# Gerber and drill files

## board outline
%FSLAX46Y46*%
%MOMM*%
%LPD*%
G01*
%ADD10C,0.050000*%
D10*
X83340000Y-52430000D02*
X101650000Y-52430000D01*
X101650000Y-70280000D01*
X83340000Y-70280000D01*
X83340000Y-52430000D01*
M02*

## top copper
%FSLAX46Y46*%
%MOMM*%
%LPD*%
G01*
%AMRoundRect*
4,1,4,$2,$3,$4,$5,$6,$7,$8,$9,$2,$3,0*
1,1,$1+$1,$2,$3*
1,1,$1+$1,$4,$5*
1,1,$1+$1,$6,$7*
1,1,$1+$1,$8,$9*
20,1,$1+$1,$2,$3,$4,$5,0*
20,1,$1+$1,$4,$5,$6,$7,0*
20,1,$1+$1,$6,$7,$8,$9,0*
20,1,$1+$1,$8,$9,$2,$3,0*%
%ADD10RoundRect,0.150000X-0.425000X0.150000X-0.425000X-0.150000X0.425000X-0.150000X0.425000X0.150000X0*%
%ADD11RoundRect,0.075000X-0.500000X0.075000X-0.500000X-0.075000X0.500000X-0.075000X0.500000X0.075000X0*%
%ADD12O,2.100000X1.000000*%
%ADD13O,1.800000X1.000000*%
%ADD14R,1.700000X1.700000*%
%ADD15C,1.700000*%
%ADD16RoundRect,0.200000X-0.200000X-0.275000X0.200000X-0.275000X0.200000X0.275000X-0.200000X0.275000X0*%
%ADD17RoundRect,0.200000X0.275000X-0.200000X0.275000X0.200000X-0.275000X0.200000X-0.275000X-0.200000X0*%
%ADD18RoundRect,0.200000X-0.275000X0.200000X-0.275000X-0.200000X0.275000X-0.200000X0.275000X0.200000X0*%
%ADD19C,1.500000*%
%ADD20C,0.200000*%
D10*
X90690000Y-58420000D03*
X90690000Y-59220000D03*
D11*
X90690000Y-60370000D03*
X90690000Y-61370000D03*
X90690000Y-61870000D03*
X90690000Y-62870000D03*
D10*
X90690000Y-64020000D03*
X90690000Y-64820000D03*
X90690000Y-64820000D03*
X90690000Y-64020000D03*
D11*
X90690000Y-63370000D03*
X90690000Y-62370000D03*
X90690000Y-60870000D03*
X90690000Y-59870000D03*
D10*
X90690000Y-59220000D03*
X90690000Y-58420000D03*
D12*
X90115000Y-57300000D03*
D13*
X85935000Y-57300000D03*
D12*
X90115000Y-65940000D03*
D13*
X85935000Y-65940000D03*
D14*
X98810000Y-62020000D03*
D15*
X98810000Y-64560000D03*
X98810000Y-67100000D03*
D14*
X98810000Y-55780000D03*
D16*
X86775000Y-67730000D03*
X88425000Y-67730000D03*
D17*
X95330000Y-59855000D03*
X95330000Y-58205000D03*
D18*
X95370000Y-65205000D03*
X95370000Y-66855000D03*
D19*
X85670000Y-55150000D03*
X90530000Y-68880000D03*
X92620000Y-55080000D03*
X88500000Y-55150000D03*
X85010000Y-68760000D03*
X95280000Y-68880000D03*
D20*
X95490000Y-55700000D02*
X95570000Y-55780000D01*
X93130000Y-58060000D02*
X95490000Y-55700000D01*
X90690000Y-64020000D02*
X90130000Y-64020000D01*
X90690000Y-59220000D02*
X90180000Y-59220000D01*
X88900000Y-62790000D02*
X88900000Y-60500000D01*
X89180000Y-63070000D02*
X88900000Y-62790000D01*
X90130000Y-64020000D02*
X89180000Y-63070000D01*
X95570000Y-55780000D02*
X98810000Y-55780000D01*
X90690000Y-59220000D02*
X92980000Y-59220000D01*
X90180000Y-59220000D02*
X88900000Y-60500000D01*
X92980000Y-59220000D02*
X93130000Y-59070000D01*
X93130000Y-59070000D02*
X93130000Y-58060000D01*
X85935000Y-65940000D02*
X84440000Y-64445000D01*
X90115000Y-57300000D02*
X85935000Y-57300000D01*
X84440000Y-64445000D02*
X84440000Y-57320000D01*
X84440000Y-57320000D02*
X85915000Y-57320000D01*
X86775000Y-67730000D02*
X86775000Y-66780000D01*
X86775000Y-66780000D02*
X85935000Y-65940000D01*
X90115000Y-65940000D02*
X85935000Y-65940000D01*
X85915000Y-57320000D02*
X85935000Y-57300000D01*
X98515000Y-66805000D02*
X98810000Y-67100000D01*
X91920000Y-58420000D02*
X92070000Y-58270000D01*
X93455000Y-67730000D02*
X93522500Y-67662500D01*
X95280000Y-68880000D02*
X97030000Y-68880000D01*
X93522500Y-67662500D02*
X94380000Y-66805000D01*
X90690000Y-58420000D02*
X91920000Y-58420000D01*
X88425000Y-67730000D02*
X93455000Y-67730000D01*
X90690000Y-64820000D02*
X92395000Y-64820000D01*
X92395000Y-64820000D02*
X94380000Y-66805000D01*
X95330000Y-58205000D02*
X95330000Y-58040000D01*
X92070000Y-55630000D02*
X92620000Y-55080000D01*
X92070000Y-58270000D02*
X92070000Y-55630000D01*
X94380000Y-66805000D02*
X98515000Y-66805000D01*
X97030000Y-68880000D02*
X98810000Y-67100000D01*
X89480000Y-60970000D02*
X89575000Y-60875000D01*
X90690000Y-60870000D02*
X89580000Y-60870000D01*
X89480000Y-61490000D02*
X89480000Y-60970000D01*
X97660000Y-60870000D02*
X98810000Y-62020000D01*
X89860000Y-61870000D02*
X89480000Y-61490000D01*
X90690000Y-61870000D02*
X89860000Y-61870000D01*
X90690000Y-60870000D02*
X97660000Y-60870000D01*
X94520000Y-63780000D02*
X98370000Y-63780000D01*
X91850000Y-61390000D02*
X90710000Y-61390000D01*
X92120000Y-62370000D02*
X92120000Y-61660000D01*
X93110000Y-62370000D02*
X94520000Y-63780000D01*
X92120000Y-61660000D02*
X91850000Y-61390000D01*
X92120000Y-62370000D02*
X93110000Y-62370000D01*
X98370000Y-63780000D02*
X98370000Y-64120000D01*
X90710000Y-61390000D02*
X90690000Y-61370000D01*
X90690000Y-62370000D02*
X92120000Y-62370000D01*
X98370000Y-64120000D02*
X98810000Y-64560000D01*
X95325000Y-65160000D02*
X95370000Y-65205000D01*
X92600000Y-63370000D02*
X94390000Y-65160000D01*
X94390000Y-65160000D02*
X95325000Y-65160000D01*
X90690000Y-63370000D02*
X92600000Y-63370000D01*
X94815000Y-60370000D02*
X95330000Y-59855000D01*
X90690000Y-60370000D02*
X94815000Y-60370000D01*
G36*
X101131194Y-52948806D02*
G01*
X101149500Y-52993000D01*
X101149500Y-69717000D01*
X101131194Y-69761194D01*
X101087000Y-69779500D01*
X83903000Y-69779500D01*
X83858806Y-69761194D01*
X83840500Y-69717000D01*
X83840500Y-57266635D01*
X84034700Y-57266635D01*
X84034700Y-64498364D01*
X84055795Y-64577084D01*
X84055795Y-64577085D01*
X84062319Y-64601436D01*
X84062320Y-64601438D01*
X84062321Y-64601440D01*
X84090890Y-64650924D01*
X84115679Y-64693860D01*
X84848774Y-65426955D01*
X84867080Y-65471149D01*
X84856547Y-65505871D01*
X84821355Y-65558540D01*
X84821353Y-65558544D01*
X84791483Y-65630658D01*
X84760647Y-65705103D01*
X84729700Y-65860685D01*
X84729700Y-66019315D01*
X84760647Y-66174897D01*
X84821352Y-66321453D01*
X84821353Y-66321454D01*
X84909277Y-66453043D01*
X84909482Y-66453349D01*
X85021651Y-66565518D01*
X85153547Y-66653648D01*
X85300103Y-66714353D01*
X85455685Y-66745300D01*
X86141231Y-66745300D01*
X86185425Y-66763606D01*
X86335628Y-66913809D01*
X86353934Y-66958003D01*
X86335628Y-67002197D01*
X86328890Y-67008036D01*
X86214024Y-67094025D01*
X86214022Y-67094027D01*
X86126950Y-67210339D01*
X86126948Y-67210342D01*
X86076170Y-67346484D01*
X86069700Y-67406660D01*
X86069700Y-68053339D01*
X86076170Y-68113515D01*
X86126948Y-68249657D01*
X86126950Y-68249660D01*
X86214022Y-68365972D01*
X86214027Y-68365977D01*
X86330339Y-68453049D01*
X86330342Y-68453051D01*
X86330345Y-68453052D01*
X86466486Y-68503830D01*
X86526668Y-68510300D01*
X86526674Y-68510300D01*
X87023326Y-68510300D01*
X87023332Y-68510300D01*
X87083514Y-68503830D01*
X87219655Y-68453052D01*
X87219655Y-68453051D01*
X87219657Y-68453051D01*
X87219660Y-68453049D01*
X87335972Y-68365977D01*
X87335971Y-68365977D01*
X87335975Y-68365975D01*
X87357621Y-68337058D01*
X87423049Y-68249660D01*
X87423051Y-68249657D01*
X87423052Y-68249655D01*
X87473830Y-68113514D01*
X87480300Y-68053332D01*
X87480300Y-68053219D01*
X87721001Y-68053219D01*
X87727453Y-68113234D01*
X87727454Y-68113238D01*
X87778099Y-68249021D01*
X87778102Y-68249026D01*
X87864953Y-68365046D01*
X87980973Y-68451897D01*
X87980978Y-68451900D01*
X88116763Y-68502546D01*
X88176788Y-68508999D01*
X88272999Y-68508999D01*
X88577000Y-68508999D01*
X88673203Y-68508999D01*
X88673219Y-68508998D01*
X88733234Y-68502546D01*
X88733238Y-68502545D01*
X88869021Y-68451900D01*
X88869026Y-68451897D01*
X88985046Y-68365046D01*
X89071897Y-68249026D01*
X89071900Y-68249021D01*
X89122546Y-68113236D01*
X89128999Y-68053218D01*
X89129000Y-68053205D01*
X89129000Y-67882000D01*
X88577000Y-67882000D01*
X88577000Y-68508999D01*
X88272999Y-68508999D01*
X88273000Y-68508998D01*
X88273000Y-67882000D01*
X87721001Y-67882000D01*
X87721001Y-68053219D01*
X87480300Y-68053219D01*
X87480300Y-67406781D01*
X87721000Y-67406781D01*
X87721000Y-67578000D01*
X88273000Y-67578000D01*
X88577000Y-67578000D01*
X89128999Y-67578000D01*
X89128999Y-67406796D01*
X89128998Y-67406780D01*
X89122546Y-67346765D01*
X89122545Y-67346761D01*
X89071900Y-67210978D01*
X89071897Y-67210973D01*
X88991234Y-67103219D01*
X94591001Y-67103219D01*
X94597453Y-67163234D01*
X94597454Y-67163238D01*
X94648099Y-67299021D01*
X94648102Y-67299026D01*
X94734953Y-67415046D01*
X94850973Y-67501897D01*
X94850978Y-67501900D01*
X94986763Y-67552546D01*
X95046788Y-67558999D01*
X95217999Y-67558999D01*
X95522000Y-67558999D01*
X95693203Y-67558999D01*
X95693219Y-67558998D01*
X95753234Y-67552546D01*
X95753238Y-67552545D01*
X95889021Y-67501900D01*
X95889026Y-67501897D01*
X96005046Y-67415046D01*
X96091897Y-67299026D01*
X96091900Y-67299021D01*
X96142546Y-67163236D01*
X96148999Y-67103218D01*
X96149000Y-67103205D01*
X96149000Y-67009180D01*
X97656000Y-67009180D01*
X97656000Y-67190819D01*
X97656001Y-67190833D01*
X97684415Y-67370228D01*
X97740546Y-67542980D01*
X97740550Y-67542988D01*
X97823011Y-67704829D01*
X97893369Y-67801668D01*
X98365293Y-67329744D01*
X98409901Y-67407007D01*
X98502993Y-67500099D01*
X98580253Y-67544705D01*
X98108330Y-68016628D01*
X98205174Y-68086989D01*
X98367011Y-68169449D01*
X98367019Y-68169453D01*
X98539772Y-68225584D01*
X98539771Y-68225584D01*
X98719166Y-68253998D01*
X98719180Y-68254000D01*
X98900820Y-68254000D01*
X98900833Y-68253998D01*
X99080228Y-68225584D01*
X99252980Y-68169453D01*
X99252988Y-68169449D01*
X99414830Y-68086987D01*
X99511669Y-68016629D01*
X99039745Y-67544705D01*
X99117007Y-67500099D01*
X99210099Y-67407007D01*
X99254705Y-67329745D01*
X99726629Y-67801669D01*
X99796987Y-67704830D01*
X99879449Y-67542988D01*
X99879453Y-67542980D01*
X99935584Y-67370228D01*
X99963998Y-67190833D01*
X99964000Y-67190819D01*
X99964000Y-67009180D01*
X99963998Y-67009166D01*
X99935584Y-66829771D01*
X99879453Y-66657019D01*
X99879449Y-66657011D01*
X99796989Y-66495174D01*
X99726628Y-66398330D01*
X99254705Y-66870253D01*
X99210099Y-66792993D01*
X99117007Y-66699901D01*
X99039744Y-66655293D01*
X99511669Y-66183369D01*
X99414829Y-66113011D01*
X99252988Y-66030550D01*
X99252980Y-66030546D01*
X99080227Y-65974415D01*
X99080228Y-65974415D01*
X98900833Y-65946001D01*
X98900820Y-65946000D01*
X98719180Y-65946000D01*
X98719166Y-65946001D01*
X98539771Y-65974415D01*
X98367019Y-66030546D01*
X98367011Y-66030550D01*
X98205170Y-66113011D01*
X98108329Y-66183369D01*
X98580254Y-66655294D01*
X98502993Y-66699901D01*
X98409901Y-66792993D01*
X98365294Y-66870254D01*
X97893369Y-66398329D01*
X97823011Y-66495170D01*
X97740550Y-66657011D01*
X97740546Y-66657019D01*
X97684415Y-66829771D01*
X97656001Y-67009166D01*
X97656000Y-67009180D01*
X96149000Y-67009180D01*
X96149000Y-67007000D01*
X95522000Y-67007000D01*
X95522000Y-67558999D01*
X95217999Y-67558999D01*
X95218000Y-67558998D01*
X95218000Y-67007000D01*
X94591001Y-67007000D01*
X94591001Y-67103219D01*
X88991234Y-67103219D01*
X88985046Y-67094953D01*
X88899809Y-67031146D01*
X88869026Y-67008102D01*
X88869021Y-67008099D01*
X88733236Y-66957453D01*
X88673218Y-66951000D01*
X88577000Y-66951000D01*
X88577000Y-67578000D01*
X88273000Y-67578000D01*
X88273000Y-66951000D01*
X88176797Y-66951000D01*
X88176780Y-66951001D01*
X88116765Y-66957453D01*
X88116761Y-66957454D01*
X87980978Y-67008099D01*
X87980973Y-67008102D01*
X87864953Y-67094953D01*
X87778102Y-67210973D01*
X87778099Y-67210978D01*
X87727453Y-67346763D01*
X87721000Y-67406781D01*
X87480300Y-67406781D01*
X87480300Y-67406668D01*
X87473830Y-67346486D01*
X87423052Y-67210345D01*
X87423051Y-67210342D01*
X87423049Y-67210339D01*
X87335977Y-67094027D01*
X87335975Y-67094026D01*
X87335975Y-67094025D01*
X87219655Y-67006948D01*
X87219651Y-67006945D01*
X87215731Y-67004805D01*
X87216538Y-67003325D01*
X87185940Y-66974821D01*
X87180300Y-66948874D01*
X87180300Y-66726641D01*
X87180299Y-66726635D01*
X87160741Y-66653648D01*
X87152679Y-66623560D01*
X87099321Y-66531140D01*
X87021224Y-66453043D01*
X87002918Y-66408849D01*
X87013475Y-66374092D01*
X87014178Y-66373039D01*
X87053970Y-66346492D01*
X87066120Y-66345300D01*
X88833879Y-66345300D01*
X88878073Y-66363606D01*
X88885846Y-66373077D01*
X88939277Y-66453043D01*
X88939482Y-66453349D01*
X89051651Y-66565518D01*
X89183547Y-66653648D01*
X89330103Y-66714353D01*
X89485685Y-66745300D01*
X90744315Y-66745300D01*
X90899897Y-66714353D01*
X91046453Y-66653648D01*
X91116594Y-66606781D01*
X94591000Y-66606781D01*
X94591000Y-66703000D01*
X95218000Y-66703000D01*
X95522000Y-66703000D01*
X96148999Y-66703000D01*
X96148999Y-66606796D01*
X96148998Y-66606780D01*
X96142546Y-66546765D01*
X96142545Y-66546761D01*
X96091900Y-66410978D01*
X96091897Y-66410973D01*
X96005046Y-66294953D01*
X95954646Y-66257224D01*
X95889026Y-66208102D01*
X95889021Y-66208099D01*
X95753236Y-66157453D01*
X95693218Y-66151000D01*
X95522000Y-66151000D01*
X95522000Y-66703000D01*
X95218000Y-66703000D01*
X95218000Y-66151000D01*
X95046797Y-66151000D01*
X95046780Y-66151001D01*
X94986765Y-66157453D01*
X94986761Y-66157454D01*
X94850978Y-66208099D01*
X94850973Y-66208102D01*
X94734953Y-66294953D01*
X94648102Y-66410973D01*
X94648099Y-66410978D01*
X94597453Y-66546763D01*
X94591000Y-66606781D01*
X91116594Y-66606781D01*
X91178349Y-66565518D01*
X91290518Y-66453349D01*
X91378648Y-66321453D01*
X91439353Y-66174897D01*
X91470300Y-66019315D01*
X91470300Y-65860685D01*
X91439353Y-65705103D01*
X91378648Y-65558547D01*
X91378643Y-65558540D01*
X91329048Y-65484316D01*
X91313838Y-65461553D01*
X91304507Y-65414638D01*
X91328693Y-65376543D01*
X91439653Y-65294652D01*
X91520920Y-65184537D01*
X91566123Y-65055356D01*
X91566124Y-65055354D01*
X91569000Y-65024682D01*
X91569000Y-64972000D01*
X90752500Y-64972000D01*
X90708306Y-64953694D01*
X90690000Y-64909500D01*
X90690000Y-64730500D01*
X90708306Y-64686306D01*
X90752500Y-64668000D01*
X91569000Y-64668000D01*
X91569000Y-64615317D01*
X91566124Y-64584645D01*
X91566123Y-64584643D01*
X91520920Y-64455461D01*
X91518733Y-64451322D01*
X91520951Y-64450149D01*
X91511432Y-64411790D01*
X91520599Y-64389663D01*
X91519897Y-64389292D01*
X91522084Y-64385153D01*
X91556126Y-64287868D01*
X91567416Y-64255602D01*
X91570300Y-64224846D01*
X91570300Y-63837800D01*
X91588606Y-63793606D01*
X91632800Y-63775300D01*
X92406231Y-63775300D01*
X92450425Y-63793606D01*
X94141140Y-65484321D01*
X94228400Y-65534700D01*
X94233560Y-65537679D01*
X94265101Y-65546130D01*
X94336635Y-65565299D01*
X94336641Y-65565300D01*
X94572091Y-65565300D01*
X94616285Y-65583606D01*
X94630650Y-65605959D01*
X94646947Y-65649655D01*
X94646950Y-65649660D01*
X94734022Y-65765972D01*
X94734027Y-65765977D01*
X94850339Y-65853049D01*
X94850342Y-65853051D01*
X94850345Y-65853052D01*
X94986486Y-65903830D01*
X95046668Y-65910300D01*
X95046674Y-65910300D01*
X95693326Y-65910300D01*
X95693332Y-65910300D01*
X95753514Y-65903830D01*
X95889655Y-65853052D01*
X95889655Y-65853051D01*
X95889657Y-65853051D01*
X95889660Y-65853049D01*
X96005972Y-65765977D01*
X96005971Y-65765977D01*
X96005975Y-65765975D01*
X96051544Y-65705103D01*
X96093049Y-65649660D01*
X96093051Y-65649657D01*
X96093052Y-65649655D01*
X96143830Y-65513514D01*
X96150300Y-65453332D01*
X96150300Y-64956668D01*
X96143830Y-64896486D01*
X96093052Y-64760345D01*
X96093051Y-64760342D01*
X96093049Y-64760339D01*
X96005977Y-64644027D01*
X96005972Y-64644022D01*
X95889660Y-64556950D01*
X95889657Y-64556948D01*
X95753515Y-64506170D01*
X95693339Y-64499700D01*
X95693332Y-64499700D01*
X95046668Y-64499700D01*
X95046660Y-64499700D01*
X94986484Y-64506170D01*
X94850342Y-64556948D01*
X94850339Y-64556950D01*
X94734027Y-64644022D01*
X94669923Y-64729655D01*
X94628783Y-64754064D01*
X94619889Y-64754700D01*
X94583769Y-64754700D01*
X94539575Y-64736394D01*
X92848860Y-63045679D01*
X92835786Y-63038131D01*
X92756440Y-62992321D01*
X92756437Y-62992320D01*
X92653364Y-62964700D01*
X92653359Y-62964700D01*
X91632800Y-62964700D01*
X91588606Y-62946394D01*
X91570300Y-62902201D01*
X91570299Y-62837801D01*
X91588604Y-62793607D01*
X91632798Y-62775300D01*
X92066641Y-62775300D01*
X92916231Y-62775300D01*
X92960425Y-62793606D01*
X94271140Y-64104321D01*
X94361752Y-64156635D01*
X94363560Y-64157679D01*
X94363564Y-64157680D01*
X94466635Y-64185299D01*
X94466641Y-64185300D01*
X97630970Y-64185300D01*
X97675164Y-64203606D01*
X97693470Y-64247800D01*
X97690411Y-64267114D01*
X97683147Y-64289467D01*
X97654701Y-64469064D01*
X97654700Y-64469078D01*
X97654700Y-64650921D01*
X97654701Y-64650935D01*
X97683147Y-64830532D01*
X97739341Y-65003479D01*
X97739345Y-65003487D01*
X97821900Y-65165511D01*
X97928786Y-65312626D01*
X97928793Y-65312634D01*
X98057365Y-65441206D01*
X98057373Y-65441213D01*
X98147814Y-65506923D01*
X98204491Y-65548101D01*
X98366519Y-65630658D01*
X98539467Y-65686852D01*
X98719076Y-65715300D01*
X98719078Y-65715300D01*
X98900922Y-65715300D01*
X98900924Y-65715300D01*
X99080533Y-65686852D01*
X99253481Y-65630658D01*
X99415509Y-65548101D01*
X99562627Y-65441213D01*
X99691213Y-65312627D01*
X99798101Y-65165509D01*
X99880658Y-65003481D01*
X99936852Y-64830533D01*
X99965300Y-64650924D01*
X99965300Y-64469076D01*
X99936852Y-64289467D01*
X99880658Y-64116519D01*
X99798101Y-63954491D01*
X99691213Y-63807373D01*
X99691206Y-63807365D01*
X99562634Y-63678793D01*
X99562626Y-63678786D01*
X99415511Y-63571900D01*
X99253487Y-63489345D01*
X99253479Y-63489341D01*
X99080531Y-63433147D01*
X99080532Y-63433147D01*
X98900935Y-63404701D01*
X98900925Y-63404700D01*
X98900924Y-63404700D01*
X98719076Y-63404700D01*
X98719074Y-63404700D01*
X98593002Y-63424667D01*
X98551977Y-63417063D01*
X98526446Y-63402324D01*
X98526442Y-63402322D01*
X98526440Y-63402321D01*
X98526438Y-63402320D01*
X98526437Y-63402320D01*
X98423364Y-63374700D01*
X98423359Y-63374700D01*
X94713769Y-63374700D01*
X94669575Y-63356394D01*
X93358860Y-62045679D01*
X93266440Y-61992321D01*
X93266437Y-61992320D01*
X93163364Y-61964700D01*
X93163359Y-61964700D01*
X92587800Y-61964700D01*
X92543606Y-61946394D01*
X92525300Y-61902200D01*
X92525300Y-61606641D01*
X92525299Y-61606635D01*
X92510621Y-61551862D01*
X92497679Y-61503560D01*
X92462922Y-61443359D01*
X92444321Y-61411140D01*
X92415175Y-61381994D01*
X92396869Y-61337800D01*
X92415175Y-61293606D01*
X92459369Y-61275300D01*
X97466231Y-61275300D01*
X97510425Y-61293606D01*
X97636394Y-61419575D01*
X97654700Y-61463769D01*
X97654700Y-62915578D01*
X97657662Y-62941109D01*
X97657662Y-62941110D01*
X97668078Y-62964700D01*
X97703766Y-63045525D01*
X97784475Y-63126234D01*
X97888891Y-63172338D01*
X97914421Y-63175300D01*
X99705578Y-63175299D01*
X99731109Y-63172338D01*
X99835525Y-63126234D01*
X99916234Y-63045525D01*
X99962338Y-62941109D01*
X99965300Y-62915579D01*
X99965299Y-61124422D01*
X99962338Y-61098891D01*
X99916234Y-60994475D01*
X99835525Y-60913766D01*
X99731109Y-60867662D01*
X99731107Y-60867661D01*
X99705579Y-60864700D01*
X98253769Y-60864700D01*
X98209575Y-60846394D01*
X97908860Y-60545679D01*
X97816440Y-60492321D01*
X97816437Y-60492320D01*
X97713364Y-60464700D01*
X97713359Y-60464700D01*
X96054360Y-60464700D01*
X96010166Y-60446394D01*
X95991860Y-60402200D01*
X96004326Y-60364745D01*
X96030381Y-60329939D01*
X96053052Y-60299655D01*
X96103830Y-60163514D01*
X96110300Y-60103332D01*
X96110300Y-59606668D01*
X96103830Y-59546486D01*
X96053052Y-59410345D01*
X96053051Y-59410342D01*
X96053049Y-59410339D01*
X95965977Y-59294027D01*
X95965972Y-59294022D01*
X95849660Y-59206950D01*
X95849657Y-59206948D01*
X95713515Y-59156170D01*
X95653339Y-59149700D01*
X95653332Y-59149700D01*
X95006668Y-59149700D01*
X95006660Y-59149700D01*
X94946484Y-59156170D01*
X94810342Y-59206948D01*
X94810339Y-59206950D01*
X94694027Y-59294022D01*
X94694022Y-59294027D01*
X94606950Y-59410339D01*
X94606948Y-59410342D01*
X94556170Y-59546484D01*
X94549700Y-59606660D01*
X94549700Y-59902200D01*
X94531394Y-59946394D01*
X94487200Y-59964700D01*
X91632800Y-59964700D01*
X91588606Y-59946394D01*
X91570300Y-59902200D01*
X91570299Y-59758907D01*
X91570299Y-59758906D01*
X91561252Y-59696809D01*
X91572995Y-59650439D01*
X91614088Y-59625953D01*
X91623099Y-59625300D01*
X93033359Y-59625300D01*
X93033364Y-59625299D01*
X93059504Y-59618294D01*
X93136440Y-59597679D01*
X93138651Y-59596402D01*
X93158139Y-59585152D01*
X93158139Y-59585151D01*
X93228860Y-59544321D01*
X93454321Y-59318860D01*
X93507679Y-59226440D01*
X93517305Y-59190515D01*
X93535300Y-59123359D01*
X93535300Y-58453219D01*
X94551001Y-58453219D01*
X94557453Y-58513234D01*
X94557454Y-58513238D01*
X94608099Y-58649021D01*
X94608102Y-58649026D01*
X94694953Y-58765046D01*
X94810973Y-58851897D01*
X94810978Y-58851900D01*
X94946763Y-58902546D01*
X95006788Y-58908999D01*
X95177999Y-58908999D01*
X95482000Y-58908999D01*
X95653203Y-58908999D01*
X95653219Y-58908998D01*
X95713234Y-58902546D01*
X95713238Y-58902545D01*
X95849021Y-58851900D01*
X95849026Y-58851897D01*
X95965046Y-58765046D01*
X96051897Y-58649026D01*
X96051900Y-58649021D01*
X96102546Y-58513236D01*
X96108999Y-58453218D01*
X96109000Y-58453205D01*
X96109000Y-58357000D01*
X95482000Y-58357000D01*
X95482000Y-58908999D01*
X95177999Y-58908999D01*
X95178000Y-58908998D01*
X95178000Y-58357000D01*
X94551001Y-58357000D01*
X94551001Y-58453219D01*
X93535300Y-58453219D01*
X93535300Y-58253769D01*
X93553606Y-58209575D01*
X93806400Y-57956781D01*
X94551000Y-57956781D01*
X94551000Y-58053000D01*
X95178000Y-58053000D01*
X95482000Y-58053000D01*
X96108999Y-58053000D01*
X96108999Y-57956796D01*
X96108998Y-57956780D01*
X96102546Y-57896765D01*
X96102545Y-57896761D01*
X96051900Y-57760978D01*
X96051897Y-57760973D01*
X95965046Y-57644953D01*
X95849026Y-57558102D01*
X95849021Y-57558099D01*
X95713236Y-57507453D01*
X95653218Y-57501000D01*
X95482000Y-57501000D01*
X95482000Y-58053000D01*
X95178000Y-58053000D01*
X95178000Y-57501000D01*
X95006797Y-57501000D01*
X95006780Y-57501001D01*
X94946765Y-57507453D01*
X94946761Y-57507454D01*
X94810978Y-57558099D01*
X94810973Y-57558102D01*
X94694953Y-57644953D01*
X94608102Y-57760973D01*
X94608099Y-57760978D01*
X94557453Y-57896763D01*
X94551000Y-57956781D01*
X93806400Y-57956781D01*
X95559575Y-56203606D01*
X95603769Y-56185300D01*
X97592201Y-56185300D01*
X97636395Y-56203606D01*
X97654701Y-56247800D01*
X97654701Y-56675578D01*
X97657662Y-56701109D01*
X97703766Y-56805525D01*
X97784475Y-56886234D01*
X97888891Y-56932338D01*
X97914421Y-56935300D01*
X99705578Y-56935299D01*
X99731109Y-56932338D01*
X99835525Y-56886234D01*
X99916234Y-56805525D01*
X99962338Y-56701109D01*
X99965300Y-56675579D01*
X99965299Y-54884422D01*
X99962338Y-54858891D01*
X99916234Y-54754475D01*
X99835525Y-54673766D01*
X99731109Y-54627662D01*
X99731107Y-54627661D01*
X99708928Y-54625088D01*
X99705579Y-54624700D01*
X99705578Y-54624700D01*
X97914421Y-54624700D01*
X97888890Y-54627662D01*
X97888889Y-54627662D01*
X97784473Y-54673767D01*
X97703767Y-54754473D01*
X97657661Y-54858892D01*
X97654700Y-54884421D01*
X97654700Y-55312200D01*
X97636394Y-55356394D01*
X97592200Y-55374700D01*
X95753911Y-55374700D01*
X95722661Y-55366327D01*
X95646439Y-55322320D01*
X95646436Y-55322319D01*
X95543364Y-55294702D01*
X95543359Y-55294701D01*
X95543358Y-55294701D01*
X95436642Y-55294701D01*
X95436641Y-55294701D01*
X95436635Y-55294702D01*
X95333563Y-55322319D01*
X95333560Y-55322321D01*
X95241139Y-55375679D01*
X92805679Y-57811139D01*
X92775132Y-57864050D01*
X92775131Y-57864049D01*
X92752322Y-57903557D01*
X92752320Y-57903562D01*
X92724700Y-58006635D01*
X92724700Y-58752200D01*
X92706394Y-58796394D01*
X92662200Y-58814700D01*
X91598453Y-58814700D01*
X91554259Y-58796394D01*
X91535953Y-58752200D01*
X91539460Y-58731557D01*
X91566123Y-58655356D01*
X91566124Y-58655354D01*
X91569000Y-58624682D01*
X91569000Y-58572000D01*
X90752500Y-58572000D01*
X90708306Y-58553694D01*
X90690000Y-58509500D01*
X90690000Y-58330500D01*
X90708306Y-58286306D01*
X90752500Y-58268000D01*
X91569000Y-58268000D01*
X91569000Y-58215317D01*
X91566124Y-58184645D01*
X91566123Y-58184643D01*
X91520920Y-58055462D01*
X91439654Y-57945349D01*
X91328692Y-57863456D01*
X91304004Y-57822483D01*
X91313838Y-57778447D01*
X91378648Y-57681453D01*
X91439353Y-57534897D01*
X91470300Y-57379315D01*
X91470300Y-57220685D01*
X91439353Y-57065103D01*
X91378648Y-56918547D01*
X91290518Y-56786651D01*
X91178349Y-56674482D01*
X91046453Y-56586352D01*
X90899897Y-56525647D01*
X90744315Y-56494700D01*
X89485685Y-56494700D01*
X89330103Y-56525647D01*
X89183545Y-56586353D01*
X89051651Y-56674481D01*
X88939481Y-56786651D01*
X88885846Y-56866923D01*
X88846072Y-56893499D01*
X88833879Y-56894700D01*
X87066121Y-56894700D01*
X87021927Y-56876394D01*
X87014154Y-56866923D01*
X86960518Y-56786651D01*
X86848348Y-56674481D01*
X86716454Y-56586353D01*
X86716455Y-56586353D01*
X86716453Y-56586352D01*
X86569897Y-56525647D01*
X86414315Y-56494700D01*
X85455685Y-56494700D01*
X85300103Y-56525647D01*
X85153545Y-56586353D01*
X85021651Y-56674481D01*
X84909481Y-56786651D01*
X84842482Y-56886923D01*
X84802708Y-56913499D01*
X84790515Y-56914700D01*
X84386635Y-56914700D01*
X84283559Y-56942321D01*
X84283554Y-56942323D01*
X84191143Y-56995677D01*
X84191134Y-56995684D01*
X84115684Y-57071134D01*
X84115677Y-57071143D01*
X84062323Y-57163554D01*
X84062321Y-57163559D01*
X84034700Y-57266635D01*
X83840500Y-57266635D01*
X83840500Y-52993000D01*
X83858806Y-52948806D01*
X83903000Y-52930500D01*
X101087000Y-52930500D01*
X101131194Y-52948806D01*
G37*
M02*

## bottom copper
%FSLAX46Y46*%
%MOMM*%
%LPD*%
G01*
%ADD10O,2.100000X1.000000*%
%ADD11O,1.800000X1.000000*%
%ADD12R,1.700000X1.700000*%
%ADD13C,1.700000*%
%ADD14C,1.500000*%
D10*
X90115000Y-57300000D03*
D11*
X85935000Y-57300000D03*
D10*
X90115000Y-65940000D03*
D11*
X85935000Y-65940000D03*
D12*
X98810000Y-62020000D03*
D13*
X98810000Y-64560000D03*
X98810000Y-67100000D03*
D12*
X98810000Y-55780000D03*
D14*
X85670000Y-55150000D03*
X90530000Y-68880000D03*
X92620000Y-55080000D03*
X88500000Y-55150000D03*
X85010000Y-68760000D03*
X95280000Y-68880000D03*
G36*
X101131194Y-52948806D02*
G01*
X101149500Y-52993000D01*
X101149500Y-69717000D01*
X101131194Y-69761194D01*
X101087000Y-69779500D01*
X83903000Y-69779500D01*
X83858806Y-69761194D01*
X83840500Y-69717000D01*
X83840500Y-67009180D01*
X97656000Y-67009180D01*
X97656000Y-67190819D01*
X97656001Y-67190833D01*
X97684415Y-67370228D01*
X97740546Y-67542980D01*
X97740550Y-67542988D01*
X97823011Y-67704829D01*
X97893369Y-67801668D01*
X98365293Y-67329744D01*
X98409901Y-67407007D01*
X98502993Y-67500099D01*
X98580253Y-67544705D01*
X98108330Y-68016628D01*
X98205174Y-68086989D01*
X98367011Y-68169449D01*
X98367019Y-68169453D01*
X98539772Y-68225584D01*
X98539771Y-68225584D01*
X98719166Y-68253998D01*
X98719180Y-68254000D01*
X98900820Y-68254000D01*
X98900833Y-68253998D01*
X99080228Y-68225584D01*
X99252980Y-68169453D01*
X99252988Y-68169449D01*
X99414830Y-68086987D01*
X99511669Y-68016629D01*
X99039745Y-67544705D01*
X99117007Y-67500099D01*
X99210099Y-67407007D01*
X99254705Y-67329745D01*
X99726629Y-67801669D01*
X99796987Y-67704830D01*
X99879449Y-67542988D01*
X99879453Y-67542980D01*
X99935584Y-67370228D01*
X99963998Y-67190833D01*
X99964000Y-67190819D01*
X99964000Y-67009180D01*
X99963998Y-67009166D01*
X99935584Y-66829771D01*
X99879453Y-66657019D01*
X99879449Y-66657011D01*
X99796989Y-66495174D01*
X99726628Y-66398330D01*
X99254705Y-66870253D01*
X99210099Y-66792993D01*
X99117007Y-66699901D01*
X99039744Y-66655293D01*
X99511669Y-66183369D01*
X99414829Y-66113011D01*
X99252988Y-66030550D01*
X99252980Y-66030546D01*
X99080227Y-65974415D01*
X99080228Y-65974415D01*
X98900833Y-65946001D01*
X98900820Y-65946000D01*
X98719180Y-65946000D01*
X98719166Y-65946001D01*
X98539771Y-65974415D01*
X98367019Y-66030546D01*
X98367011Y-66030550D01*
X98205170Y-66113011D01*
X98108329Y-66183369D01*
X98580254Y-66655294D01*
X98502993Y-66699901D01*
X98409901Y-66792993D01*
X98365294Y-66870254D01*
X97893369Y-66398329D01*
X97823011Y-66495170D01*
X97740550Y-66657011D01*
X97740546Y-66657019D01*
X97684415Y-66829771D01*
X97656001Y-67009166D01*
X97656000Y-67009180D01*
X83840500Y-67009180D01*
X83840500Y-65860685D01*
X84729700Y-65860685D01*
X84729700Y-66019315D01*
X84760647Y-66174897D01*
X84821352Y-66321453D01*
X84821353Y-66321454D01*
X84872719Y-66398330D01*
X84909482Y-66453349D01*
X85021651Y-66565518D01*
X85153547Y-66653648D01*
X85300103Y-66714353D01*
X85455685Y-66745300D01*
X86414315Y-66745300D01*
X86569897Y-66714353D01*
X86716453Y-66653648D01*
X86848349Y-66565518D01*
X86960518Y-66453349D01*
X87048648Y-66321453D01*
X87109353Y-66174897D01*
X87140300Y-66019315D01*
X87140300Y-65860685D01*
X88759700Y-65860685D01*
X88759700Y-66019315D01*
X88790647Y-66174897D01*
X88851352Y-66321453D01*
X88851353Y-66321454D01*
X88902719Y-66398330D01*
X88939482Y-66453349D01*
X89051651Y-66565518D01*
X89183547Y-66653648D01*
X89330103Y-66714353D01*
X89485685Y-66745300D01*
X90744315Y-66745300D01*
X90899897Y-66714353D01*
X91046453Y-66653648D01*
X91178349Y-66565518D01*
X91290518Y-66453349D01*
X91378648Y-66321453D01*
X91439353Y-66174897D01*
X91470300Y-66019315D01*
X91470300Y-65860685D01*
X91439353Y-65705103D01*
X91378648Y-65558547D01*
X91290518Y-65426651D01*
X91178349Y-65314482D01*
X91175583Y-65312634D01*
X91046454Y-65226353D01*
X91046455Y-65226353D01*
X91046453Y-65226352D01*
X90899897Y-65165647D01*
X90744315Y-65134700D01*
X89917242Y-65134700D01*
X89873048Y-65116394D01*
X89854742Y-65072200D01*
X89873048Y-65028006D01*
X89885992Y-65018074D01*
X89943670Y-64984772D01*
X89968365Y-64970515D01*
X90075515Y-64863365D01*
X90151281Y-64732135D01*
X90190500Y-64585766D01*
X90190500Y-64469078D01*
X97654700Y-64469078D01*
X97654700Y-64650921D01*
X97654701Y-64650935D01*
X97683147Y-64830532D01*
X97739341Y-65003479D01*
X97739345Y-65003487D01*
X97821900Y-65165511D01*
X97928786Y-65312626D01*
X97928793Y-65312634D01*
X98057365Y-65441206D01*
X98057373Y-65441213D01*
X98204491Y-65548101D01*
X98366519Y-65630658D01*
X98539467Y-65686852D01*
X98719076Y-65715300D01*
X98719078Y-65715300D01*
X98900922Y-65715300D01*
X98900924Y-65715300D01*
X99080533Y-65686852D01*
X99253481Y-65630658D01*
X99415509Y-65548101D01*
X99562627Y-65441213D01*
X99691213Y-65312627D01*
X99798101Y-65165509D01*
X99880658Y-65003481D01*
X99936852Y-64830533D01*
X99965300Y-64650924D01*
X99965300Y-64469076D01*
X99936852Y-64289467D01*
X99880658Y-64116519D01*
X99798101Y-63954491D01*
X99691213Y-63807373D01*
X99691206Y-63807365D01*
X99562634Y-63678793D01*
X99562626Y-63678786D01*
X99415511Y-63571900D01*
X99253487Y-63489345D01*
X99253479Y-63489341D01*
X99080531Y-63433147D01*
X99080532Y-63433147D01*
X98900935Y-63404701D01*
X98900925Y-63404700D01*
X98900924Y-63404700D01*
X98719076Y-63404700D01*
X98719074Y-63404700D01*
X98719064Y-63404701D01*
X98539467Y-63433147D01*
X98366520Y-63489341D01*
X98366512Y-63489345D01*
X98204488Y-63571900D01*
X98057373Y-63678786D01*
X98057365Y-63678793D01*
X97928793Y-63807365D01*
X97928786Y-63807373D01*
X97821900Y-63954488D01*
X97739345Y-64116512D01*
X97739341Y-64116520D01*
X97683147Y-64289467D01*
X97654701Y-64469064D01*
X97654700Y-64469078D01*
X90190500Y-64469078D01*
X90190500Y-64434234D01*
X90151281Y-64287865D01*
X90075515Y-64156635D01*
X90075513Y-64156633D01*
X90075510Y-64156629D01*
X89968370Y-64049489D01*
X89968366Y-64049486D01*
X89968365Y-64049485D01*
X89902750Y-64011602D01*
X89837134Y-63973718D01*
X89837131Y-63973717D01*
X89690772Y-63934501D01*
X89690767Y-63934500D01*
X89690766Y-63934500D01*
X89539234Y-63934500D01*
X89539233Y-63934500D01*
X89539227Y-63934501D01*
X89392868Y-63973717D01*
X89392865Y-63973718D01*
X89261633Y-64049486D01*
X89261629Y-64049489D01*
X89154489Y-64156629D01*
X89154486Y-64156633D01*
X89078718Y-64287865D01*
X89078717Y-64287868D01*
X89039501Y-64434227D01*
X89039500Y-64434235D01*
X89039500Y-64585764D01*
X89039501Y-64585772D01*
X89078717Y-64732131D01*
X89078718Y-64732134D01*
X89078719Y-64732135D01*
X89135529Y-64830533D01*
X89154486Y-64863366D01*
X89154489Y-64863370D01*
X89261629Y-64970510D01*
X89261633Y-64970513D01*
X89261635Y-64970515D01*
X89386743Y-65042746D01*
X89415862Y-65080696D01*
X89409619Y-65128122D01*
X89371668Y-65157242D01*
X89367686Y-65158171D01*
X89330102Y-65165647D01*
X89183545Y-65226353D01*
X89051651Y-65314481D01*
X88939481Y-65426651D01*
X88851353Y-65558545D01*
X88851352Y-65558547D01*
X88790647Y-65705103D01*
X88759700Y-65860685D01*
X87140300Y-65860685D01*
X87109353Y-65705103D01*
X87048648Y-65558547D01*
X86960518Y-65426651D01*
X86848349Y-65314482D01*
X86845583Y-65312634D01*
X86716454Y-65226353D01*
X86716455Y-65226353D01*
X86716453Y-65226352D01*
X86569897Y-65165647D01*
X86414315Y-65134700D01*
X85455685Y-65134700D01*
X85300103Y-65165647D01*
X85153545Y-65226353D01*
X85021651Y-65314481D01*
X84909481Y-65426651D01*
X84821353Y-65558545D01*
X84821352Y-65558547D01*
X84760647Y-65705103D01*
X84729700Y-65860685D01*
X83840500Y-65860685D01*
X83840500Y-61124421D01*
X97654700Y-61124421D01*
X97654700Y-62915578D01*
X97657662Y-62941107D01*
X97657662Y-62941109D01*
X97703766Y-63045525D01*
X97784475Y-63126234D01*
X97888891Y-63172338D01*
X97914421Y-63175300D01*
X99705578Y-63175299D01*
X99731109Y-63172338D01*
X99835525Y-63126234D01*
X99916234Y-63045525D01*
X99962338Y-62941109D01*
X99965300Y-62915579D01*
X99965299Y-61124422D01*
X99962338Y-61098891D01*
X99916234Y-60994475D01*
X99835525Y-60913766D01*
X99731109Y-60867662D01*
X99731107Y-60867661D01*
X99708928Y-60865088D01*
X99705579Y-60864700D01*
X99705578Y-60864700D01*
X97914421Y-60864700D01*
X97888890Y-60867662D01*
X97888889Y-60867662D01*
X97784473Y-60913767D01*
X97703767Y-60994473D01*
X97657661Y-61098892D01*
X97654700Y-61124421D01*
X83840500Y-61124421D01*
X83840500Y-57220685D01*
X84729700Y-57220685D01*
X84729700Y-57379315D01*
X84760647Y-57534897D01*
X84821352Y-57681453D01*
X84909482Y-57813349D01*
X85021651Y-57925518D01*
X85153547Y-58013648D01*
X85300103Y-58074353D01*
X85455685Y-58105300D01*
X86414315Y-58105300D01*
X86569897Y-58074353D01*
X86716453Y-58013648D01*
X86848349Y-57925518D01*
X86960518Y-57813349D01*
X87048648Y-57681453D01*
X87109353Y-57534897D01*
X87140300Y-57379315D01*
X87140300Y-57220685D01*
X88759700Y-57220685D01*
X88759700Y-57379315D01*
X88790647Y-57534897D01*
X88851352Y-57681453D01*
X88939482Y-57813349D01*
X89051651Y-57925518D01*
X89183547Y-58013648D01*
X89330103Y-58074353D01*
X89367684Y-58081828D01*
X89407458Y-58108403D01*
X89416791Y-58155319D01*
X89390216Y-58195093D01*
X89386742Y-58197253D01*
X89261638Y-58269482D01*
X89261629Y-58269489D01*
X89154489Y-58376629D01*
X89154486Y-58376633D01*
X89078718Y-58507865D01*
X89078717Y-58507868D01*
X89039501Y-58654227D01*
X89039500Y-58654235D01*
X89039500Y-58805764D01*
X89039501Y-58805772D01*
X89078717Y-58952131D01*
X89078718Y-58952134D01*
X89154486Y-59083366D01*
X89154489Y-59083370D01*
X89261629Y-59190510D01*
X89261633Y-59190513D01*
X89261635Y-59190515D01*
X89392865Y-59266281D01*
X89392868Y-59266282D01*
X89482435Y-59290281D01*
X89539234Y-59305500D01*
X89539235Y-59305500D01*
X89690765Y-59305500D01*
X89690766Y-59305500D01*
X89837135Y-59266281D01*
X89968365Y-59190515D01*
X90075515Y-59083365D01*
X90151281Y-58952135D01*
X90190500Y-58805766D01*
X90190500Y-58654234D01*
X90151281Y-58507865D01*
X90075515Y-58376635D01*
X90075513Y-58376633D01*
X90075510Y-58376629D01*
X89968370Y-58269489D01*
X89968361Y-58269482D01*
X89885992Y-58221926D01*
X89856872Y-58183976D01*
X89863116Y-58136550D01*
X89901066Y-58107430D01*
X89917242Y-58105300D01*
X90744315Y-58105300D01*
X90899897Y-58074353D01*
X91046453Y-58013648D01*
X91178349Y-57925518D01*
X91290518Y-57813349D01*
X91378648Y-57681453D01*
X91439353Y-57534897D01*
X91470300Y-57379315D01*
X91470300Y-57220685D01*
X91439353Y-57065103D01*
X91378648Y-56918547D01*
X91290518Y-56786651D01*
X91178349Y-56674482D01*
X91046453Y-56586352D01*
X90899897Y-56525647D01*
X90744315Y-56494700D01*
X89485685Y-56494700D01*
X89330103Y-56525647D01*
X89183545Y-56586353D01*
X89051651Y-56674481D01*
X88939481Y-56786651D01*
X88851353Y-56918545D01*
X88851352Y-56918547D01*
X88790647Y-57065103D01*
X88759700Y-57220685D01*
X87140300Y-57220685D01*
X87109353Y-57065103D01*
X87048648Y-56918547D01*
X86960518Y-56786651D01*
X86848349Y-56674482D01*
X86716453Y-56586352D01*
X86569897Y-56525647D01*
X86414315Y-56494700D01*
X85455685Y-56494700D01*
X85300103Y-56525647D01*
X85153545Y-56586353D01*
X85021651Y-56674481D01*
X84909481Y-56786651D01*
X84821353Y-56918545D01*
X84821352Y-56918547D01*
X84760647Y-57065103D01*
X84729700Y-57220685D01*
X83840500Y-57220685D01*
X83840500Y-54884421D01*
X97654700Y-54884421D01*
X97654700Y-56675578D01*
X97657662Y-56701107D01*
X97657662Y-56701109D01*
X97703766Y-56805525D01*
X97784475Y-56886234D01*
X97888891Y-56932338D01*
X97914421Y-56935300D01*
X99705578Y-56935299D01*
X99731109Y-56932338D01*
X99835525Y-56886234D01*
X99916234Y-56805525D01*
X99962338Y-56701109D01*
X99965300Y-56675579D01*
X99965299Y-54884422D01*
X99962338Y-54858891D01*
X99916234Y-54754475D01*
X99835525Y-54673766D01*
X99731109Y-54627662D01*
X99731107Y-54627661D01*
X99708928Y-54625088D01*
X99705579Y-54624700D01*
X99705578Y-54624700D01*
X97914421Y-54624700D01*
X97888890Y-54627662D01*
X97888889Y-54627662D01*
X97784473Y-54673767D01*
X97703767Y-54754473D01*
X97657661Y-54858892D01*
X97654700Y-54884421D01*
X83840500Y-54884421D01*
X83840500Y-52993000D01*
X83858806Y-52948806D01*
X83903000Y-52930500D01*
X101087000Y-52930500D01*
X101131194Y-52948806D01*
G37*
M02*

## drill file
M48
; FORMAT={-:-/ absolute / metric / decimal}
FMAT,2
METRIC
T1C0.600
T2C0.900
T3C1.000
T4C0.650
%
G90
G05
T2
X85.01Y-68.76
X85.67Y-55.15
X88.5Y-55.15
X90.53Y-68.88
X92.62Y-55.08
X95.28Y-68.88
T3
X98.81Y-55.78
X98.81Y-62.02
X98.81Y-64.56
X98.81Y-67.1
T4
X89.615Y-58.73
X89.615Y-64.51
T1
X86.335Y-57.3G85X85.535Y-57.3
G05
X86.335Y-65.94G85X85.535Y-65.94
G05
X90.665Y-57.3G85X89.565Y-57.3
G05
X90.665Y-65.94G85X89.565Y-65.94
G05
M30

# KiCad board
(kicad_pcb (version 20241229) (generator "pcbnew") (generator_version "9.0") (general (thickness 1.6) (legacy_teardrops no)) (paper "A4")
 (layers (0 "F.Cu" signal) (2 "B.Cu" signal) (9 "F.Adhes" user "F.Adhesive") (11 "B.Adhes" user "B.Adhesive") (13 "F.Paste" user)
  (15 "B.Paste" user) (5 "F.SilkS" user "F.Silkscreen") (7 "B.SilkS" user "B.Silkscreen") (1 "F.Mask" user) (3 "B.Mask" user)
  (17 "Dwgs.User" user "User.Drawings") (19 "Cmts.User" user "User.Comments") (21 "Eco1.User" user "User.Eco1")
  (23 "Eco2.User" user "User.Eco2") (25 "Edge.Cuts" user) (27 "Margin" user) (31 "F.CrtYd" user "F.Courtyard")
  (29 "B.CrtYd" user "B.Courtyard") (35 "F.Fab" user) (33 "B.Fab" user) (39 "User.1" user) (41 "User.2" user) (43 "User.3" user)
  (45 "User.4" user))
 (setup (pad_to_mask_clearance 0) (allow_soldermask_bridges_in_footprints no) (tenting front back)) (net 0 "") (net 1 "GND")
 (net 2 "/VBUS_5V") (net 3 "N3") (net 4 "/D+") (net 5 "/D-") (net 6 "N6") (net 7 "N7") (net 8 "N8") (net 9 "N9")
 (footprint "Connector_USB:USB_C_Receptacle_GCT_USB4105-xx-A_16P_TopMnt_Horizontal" (layer "F.Cu") (at 87.01 61.62 -90)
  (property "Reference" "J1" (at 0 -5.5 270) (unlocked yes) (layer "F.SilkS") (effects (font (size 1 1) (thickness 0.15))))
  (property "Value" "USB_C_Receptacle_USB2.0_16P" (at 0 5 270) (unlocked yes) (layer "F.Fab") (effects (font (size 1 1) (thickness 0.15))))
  (pad "" np_thru_hole circle (at -2.89 -2.605 270) (size 0.65 0.65) (drill 0.65) (layers "*.Cu" "*.Mask"))
  (pad "" np_thru_hole circle (at 2.89 -2.605 270) (size 0.65 0.65) (drill 0.65) (layers "*.Cu" "*.Mask"))
  (pad "A1" smd roundrect (at -3.2 -3.68 270) (size 0.6 1.15) (layers "F.Cu" "F.Mask" "F.Paste") (roundrect_rratio 0.25) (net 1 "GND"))
  (pad "A4" smd roundrect (at -2.4 -3.68 270) (size 0.6 1.15) (layers "F.Cu" "F.Mask" "F.Paste") (roundrect_rratio 0.25) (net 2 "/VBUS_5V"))
  (pad "A5" smd roundrect (at -1.25 -3.68 270) (size 0.3 1.15) (layers "F.Cu" "F.Mask" "F.Paste") (roundrect_rratio 0.25) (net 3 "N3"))
  (pad "A6" smd roundrect (at -0.25 -3.68 270) (size 0.3 1.15) (layers "F.Cu" "F.Mask" "F.Paste") (roundrect_rratio 0.25) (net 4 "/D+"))
  (pad "A7" smd roundrect (at 0.25 -3.68 270) (size 0.3 1.15) (layers "F.Cu" "F.Mask" "F.Paste") (roundrect_rratio 0.25) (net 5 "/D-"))
  (pad "A8" smd roundrect (at 1.25 -3.68 270) (size 0.3 1.15) (layers "F.Cu" "F.Mask" "F.Paste") (roundrect_rratio 0.25) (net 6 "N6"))
  (pad "A9" smd roundrect (at 2.4 -3.68 270) (size 0.6 1.15) (layers "F.Cu" "F.Mask" "F.Paste") (roundrect_rratio 0.25) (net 2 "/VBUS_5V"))
  (pad "A12" smd roundrect (at 3.2 -3.68 270) (size 0.6 1.15) (layers "F.Cu" "F.Mask" "F.Paste") (roundrect_rratio 0.25) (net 1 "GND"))
  (pad "B1" smd roundrect (at 3.2 -3.68 270) (size 0.6 1.15) (layers "F.Cu" "F.Mask" "F.Paste") (roundrect_rratio 0.25) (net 1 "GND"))
  (pad "B4" smd roundrect (at 2.4 -3.68 270) (size 0.6 1.15) (layers "F.Cu" "F.Mask" "F.Paste") (roundrect_rratio 0.25) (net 2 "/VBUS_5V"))
  (pad "B5" smd roundrect (at 1.75 -3.68 270) (size 0.3 1.15) (layers "F.Cu" "F.Mask" "F.Paste") (roundrect_rratio 0.25) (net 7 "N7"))
  (pad "B6" smd roundrect (at 0.75 -3.68 270) (size 0.3 1.15) (layers "F.Cu" "F.Mask" "F.Paste") (roundrect_rratio 0.25) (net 4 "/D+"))
  (pad "B7" smd roundrect (at -0.75 -3.68 270) (size 0.3 1.15) (layers "F.Cu" "F.Mask" "F.Paste") (roundrect_rratio 0.25) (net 5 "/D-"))
  (pad "B8" smd roundrect (at -1.75 -3.68 270) (size 0.3 1.15) (layers "F.Cu" "F.Mask" "F.Paste") (roundrect_rratio 0.25) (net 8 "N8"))
  (pad "B9" smd roundrect (at -2.4 -3.68 270) (size 0.6 1.15) (layers "F.Cu" "F.Mask" "F.Paste") (roundrect_rratio 0.25) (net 2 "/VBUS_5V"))
  (pad "B12" smd roundrect (at -3.2 -3.68 270) (size 0.6 1.15) (layers "F.Cu" "F.Mask" "F.Paste") (roundrect_rratio 0.25) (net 1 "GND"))
  (pad "S1" thru_hole oval (at -4.32 -3.105 270) (size 1 2.1) (drill oval 0.6 1.7) (layers "*.Cu" "*.Mask" "F.Paste")
   (remove_unused_layers no) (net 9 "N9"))
  (pad "S1" thru_hole oval (at -4.32 1.075 270) (size 1 1.8) (drill oval 0.6 1.4) (layers "*.Cu" "*.Mask" "F.Paste")
   (remove_unused_layers no) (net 9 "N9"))
  (pad "S1" thru_hole oval (at 4.32 -3.105 270) (size 1 2.1) (drill oval 0.6 1.7) (layers "*.Cu" "*.Mask" "F.Paste")
   (remove_unused_layers no) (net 9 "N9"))
  (pad "S1" thru_hole oval (at 4.32 1.075 270) (size 1 1.8) (drill oval 0.6 1.4) (layers "*.Cu" "*.Mask" "F.Paste")
   (remove_unused_layers no) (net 9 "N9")))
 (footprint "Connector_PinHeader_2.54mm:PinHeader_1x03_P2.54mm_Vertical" (layer "F.Cu") (at 98.81 62.02)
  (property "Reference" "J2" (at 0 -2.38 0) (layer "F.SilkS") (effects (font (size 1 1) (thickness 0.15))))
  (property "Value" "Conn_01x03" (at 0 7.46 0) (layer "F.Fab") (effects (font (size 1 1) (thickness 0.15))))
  (pad "1" thru_hole rect (at 0 0) (size 1.7 1.7) (drill 1) (layers "*.Cu" "*.Mask") (remove_unused_layers no) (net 5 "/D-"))
  (pad "2" thru_hole circle (at 0 2.54) (size 1.7 1.7) (drill 1) (layers "*.Cu" "*.Mask") (remove_unused_layers no) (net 4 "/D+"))
  (pad "3" thru_hole circle (at 0 5.08) (size 1.7 1.7) (drill 1) (layers "*.Cu" "*.Mask") (remove_unused_layers no) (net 1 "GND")))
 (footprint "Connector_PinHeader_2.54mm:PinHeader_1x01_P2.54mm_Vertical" (layer "F.Cu") (at 98.81 55.78)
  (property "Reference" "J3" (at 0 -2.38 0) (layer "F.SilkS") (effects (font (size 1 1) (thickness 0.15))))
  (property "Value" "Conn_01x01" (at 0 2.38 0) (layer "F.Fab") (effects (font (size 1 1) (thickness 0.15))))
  (pad "1" thru_hole rect (at 0 0) (size 1.7 1.7) (drill 1) (layers "*.Cu" "*.Mask") (remove_unused_layers no) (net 2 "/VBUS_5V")))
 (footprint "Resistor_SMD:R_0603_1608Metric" (layer "F.Cu") (at 87.6 67.73)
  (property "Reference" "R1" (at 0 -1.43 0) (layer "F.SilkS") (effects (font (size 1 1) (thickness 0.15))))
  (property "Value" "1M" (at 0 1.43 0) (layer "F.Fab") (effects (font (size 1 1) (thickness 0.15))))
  (pad "1" smd roundrect (at -0.825 0) (size 0.8 0.95) (layers "F.Cu" "F.Mask" "F.Paste") (roundrect_rratio 0.25) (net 9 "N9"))
  (pad "2" smd roundrect (at 0.825 0) (size 0.8 0.95) (layers "F.Cu" "F.Mask" "F.Paste") (roundrect_rratio 0.25) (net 1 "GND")))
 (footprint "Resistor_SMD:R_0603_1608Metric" (layer "F.Cu") (at 95.33 59.03 90)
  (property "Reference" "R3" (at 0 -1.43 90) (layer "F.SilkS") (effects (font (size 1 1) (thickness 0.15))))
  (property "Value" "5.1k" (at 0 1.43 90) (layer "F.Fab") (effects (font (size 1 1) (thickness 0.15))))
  (pad "1" smd roundrect (at -0.825 0 90) (size 0.8 0.95) (layers "F.Cu" "F.Mask" "F.Paste") (roundrect_rratio 0.25) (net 3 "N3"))
  (pad "2" smd roundrect (at 0.825 0 90) (size 0.8 0.95) (layers "F.Cu" "F.Mask" "F.Paste") (roundrect_rratio 0.25) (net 1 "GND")))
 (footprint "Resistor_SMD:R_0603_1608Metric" (layer "F.Cu") (at 95.37 66.03 -90)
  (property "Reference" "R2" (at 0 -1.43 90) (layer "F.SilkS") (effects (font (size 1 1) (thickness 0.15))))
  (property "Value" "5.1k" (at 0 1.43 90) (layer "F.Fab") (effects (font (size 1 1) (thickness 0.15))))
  (pad "1" smd roundrect (at -0.825 0 270) (size 0.8 0.95) (layers "F.Cu" "F.Mask" "F.Paste") (roundrect_rratio 0.25) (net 7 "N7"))
  (pad "2" smd roundrect (at 0.825 0 270) (size 0.8 0.95) (layers "F.Cu" "F.Mask" "F.Paste") (roundrect_rratio 0.25) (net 1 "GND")))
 (gr_rect (start 83.34 52.43) (end 101.65 70.28) (stroke (width 0.05) (type default)) (fill no) (layer "Edge.Cuts"))
 (segment (start 95.49 55.7) (end 95.57 55.78) (width 0.2) (layer "F.Cu") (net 2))
 (segment (start 93.13 58.06) (end 95.49 55.7) (width 0.2) (layer "F.Cu") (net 2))
 (segment (start 90.69 64.02) (end 90.13 64.02) (width 0.2) (layer "F.Cu") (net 2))
 (segment (start 90.69 59.22) (end 90.18 59.22) (width 0.2) (layer "F.Cu") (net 2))
 (segment (start 88.9 62.79) (end 88.9 60.5) (width 0.2) (layer "F.Cu") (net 2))
 (segment (start 89.18 63.07) (end 88.9 62.79) (width 0.2) (layer "F.Cu") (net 2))
 (segment (start 90.13 64.02) (end 89.18 63.07) (width 0.2) (layer "F.Cu") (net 2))
 (segment (start 95.57 55.78) (end 98.81 55.78) (width 0.2) (layer "F.Cu") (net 2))
 (segment (start 90.69 59.22) (end 92.98 59.22) (width 0.2) (layer "F.Cu") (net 2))
 (segment (start 90.18 59.22) (end 88.9 60.5) (width 0.2) (layer "F.Cu") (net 2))
 (segment (start 92.98 59.22) (end 93.13 59.07) (width 0.2) (layer "F.Cu") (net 2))
 (segment (start 93.13 59.07) (end 93.13 58.06) (width 0.2) (layer "F.Cu") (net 2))
 (segment (start 85.935 65.94) (end 84.44 64.445) (width 0.2) (layer "F.Cu") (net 9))
 (segment (start 90.115 57.3) (end 85.935 57.3) (width 0.2) (layer "F.Cu") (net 9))
 (segment (start 84.44 64.445) (end 84.44 57.32) (width 0.2) (layer "F.Cu") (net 9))
 (segment (start 84.44 57.32) (end 85.915 57.32) (width 0.2) (layer "F.Cu") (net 9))
 (segment (start 86.775 67.73) (end 86.775 66.78) (width 0.2) (layer "F.Cu") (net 9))
 (segment (start 86.775 66.78) (end 85.935 65.94) (width 0.2) (layer "F.Cu") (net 9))
 (segment (start 90.115 65.94) (end 85.935 65.94) (width 0.2) (layer "F.Cu") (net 9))
 (segment (start 85.915 57.32) (end 85.935 57.3) (width 0.2) (layer "F.Cu") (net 9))
 (segment (start 98.515 66.805) (end 98.81 67.1) (width 0.2) (layer "F.Cu") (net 1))
 (segment (start 91.92 58.42) (end 92.07 58.27) (width 0.2) (layer "F.Cu") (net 1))
 (segment (start 93.455 67.73) (end 93.5225 67.6625) (width 0.2) (layer "F.Cu") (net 1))
 (segment (start 95.28 68.88) (end 97.03 68.88) (width 0.2) (layer "F.Cu") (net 1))
 (segment (start 93.5225 67.6625) (end 94.38 66.805) (width 0.2) (layer "F.Cu") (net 1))
 (segment (start 90.69 58.42) (end 91.92 58.42) (width 0.2) (layer "F.Cu") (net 1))
 (segment (start 88.425 67.73) (end 93.455 67.73) (width 0.2) (layer "F.Cu") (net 1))
 (segment (start 90.69 64.82) (end 92.395 64.82) (width 0.2) (layer "F.Cu") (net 1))
 (segment (start 92.395 64.82) (end 94.38 66.805) (width 0.2) (layer "F.Cu") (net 1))
 (segment (start 95.33 58.205) (end 95.33 58.04) (width 0.2) (layer "F.Cu") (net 1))
 (segment (start 92.07 55.63) (end 92.62 55.08) (width 0.2) (layer "F.Cu") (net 1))
 (segment (start 92.07 58.27) (end 92.07 55.63) (width 0.2) (layer "F.Cu") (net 1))
 (segment (start 94.38 66.805) (end 98.515 66.805) (width 0.2) (layer "F.Cu") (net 1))
 (segment (start 97.03 68.88) (end 98.81 67.1) (width 0.2) (layer "F.Cu") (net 1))
 (via (at 85.67 55.15) (size 1.5) (drill 0.9) (layers "F.Cu" "B.Cu") (free yes) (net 1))
 (via (at 90.53 68.88) (size 1.5) (drill 0.9) (layers "F.Cu" "B.Cu") (free yes) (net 1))
 (via (at 92.62 55.08) (size 1.5) (drill 0.9) (layers "F.Cu" "B.Cu") (free yes) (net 1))
 (via (at 88.5 55.15) (size 1.5) (drill 0.9) (layers "F.Cu" "B.Cu") (free yes) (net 1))
 (via (at 85.01 68.76) (size 1.5) (drill 0.9) (layers "F.Cu" "B.Cu") (free yes) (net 1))
 (via (at 95.28 68.88) (size 1.5) (drill 0.9) (layers "F.Cu" "B.Cu") (free yes) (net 1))
 (segment (start 89.48 60.97) (end 89.575 60.875) (width 0.2) (layer "F.Cu") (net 5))
 (segment (start 90.69 60.87) (end 89.58 60.87) (width 0.2) (layer "F.Cu") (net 5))
 (segment (start 89.48 61.49) (end 89.48 60.97) (width 0.2) (layer "F.Cu") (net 5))
 (segment (start 97.66 60.87) (end 98.81 62.02) (width 0.2) (layer "F.Cu") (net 5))
 (segment (start 89.86 61.87) (end 89.48 61.49) (width 0.2) (layer "F.Cu") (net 5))
 (segment (start 90.69 61.87) (end 89.86 61.87) (width 0.2) (layer "F.Cu") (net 5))
 (segment (start 90.69 60.87) (end 97.66 60.87) (width 0.2) (layer "F.Cu") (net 5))
 (segment (start 94.52 63.78) (end 98.37 63.78) (width 0.2) (layer "F.Cu") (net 4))
 (segment (start 91.85 61.39) (end 90.71 61.39) (width 0.2) (layer "F.Cu") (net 4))
 (segment (start 92.12 62.37) (end 92.12 61.66) (width 0.2) (layer "F.Cu") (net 4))
 (segment (start 93.11 62.37) (end 94.52 63.78) (width 0.2) (layer "F.Cu") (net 4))
 (segment (start 92.12 61.66) (end 91.85 61.39) (width 0.2) (layer "F.Cu") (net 4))
 (segment (start 92.12 62.37) (end 93.11 62.37) (width 0.2) (layer "F.Cu") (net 4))
 (segment (start 98.37 63.78) (end 98.37 64.12) (width 0.2) (layer "F.Cu") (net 4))
 (segment (start 90.71 61.39) (end 90.69 61.37) (width 0.2) (layer "F.Cu") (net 4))
 (segment (start 90.69 62.37) (end 92.12 62.37) (width 0.2) (layer "F.Cu") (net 4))
 (segment (start 98.37 64.12) (end 98.81 64.56) (width 0.2) (layer "F.Cu") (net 4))
 (segment (start 95.325 65.16) (end 95.37 65.205) (width 0.2) (layer "F.Cu") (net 7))
 (segment (start 92.6 63.37) (end 94.39 65.16) (width 0.2) (layer "F.Cu") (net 7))
 (segment (start 94.39 65.16) (end 95.325 65.16) (width 0.2) (layer "F.Cu") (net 7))
 (segment (start 90.69 63.37) (end 92.6 63.37) (width 0.2) (layer "F.Cu") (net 7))
 (segment (start 94.815 60.37) (end 95.33 59.855) (width 0.2) (layer "F.Cu") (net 3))
 (segment (start 90.69 60.37) (end 94.815 60.37) (width 0.2) (layer "F.Cu") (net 3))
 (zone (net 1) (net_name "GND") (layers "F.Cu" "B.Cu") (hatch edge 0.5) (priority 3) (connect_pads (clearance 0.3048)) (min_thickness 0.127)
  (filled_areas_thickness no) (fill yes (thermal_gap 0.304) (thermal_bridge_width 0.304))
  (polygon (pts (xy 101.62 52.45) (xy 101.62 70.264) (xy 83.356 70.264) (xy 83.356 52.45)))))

